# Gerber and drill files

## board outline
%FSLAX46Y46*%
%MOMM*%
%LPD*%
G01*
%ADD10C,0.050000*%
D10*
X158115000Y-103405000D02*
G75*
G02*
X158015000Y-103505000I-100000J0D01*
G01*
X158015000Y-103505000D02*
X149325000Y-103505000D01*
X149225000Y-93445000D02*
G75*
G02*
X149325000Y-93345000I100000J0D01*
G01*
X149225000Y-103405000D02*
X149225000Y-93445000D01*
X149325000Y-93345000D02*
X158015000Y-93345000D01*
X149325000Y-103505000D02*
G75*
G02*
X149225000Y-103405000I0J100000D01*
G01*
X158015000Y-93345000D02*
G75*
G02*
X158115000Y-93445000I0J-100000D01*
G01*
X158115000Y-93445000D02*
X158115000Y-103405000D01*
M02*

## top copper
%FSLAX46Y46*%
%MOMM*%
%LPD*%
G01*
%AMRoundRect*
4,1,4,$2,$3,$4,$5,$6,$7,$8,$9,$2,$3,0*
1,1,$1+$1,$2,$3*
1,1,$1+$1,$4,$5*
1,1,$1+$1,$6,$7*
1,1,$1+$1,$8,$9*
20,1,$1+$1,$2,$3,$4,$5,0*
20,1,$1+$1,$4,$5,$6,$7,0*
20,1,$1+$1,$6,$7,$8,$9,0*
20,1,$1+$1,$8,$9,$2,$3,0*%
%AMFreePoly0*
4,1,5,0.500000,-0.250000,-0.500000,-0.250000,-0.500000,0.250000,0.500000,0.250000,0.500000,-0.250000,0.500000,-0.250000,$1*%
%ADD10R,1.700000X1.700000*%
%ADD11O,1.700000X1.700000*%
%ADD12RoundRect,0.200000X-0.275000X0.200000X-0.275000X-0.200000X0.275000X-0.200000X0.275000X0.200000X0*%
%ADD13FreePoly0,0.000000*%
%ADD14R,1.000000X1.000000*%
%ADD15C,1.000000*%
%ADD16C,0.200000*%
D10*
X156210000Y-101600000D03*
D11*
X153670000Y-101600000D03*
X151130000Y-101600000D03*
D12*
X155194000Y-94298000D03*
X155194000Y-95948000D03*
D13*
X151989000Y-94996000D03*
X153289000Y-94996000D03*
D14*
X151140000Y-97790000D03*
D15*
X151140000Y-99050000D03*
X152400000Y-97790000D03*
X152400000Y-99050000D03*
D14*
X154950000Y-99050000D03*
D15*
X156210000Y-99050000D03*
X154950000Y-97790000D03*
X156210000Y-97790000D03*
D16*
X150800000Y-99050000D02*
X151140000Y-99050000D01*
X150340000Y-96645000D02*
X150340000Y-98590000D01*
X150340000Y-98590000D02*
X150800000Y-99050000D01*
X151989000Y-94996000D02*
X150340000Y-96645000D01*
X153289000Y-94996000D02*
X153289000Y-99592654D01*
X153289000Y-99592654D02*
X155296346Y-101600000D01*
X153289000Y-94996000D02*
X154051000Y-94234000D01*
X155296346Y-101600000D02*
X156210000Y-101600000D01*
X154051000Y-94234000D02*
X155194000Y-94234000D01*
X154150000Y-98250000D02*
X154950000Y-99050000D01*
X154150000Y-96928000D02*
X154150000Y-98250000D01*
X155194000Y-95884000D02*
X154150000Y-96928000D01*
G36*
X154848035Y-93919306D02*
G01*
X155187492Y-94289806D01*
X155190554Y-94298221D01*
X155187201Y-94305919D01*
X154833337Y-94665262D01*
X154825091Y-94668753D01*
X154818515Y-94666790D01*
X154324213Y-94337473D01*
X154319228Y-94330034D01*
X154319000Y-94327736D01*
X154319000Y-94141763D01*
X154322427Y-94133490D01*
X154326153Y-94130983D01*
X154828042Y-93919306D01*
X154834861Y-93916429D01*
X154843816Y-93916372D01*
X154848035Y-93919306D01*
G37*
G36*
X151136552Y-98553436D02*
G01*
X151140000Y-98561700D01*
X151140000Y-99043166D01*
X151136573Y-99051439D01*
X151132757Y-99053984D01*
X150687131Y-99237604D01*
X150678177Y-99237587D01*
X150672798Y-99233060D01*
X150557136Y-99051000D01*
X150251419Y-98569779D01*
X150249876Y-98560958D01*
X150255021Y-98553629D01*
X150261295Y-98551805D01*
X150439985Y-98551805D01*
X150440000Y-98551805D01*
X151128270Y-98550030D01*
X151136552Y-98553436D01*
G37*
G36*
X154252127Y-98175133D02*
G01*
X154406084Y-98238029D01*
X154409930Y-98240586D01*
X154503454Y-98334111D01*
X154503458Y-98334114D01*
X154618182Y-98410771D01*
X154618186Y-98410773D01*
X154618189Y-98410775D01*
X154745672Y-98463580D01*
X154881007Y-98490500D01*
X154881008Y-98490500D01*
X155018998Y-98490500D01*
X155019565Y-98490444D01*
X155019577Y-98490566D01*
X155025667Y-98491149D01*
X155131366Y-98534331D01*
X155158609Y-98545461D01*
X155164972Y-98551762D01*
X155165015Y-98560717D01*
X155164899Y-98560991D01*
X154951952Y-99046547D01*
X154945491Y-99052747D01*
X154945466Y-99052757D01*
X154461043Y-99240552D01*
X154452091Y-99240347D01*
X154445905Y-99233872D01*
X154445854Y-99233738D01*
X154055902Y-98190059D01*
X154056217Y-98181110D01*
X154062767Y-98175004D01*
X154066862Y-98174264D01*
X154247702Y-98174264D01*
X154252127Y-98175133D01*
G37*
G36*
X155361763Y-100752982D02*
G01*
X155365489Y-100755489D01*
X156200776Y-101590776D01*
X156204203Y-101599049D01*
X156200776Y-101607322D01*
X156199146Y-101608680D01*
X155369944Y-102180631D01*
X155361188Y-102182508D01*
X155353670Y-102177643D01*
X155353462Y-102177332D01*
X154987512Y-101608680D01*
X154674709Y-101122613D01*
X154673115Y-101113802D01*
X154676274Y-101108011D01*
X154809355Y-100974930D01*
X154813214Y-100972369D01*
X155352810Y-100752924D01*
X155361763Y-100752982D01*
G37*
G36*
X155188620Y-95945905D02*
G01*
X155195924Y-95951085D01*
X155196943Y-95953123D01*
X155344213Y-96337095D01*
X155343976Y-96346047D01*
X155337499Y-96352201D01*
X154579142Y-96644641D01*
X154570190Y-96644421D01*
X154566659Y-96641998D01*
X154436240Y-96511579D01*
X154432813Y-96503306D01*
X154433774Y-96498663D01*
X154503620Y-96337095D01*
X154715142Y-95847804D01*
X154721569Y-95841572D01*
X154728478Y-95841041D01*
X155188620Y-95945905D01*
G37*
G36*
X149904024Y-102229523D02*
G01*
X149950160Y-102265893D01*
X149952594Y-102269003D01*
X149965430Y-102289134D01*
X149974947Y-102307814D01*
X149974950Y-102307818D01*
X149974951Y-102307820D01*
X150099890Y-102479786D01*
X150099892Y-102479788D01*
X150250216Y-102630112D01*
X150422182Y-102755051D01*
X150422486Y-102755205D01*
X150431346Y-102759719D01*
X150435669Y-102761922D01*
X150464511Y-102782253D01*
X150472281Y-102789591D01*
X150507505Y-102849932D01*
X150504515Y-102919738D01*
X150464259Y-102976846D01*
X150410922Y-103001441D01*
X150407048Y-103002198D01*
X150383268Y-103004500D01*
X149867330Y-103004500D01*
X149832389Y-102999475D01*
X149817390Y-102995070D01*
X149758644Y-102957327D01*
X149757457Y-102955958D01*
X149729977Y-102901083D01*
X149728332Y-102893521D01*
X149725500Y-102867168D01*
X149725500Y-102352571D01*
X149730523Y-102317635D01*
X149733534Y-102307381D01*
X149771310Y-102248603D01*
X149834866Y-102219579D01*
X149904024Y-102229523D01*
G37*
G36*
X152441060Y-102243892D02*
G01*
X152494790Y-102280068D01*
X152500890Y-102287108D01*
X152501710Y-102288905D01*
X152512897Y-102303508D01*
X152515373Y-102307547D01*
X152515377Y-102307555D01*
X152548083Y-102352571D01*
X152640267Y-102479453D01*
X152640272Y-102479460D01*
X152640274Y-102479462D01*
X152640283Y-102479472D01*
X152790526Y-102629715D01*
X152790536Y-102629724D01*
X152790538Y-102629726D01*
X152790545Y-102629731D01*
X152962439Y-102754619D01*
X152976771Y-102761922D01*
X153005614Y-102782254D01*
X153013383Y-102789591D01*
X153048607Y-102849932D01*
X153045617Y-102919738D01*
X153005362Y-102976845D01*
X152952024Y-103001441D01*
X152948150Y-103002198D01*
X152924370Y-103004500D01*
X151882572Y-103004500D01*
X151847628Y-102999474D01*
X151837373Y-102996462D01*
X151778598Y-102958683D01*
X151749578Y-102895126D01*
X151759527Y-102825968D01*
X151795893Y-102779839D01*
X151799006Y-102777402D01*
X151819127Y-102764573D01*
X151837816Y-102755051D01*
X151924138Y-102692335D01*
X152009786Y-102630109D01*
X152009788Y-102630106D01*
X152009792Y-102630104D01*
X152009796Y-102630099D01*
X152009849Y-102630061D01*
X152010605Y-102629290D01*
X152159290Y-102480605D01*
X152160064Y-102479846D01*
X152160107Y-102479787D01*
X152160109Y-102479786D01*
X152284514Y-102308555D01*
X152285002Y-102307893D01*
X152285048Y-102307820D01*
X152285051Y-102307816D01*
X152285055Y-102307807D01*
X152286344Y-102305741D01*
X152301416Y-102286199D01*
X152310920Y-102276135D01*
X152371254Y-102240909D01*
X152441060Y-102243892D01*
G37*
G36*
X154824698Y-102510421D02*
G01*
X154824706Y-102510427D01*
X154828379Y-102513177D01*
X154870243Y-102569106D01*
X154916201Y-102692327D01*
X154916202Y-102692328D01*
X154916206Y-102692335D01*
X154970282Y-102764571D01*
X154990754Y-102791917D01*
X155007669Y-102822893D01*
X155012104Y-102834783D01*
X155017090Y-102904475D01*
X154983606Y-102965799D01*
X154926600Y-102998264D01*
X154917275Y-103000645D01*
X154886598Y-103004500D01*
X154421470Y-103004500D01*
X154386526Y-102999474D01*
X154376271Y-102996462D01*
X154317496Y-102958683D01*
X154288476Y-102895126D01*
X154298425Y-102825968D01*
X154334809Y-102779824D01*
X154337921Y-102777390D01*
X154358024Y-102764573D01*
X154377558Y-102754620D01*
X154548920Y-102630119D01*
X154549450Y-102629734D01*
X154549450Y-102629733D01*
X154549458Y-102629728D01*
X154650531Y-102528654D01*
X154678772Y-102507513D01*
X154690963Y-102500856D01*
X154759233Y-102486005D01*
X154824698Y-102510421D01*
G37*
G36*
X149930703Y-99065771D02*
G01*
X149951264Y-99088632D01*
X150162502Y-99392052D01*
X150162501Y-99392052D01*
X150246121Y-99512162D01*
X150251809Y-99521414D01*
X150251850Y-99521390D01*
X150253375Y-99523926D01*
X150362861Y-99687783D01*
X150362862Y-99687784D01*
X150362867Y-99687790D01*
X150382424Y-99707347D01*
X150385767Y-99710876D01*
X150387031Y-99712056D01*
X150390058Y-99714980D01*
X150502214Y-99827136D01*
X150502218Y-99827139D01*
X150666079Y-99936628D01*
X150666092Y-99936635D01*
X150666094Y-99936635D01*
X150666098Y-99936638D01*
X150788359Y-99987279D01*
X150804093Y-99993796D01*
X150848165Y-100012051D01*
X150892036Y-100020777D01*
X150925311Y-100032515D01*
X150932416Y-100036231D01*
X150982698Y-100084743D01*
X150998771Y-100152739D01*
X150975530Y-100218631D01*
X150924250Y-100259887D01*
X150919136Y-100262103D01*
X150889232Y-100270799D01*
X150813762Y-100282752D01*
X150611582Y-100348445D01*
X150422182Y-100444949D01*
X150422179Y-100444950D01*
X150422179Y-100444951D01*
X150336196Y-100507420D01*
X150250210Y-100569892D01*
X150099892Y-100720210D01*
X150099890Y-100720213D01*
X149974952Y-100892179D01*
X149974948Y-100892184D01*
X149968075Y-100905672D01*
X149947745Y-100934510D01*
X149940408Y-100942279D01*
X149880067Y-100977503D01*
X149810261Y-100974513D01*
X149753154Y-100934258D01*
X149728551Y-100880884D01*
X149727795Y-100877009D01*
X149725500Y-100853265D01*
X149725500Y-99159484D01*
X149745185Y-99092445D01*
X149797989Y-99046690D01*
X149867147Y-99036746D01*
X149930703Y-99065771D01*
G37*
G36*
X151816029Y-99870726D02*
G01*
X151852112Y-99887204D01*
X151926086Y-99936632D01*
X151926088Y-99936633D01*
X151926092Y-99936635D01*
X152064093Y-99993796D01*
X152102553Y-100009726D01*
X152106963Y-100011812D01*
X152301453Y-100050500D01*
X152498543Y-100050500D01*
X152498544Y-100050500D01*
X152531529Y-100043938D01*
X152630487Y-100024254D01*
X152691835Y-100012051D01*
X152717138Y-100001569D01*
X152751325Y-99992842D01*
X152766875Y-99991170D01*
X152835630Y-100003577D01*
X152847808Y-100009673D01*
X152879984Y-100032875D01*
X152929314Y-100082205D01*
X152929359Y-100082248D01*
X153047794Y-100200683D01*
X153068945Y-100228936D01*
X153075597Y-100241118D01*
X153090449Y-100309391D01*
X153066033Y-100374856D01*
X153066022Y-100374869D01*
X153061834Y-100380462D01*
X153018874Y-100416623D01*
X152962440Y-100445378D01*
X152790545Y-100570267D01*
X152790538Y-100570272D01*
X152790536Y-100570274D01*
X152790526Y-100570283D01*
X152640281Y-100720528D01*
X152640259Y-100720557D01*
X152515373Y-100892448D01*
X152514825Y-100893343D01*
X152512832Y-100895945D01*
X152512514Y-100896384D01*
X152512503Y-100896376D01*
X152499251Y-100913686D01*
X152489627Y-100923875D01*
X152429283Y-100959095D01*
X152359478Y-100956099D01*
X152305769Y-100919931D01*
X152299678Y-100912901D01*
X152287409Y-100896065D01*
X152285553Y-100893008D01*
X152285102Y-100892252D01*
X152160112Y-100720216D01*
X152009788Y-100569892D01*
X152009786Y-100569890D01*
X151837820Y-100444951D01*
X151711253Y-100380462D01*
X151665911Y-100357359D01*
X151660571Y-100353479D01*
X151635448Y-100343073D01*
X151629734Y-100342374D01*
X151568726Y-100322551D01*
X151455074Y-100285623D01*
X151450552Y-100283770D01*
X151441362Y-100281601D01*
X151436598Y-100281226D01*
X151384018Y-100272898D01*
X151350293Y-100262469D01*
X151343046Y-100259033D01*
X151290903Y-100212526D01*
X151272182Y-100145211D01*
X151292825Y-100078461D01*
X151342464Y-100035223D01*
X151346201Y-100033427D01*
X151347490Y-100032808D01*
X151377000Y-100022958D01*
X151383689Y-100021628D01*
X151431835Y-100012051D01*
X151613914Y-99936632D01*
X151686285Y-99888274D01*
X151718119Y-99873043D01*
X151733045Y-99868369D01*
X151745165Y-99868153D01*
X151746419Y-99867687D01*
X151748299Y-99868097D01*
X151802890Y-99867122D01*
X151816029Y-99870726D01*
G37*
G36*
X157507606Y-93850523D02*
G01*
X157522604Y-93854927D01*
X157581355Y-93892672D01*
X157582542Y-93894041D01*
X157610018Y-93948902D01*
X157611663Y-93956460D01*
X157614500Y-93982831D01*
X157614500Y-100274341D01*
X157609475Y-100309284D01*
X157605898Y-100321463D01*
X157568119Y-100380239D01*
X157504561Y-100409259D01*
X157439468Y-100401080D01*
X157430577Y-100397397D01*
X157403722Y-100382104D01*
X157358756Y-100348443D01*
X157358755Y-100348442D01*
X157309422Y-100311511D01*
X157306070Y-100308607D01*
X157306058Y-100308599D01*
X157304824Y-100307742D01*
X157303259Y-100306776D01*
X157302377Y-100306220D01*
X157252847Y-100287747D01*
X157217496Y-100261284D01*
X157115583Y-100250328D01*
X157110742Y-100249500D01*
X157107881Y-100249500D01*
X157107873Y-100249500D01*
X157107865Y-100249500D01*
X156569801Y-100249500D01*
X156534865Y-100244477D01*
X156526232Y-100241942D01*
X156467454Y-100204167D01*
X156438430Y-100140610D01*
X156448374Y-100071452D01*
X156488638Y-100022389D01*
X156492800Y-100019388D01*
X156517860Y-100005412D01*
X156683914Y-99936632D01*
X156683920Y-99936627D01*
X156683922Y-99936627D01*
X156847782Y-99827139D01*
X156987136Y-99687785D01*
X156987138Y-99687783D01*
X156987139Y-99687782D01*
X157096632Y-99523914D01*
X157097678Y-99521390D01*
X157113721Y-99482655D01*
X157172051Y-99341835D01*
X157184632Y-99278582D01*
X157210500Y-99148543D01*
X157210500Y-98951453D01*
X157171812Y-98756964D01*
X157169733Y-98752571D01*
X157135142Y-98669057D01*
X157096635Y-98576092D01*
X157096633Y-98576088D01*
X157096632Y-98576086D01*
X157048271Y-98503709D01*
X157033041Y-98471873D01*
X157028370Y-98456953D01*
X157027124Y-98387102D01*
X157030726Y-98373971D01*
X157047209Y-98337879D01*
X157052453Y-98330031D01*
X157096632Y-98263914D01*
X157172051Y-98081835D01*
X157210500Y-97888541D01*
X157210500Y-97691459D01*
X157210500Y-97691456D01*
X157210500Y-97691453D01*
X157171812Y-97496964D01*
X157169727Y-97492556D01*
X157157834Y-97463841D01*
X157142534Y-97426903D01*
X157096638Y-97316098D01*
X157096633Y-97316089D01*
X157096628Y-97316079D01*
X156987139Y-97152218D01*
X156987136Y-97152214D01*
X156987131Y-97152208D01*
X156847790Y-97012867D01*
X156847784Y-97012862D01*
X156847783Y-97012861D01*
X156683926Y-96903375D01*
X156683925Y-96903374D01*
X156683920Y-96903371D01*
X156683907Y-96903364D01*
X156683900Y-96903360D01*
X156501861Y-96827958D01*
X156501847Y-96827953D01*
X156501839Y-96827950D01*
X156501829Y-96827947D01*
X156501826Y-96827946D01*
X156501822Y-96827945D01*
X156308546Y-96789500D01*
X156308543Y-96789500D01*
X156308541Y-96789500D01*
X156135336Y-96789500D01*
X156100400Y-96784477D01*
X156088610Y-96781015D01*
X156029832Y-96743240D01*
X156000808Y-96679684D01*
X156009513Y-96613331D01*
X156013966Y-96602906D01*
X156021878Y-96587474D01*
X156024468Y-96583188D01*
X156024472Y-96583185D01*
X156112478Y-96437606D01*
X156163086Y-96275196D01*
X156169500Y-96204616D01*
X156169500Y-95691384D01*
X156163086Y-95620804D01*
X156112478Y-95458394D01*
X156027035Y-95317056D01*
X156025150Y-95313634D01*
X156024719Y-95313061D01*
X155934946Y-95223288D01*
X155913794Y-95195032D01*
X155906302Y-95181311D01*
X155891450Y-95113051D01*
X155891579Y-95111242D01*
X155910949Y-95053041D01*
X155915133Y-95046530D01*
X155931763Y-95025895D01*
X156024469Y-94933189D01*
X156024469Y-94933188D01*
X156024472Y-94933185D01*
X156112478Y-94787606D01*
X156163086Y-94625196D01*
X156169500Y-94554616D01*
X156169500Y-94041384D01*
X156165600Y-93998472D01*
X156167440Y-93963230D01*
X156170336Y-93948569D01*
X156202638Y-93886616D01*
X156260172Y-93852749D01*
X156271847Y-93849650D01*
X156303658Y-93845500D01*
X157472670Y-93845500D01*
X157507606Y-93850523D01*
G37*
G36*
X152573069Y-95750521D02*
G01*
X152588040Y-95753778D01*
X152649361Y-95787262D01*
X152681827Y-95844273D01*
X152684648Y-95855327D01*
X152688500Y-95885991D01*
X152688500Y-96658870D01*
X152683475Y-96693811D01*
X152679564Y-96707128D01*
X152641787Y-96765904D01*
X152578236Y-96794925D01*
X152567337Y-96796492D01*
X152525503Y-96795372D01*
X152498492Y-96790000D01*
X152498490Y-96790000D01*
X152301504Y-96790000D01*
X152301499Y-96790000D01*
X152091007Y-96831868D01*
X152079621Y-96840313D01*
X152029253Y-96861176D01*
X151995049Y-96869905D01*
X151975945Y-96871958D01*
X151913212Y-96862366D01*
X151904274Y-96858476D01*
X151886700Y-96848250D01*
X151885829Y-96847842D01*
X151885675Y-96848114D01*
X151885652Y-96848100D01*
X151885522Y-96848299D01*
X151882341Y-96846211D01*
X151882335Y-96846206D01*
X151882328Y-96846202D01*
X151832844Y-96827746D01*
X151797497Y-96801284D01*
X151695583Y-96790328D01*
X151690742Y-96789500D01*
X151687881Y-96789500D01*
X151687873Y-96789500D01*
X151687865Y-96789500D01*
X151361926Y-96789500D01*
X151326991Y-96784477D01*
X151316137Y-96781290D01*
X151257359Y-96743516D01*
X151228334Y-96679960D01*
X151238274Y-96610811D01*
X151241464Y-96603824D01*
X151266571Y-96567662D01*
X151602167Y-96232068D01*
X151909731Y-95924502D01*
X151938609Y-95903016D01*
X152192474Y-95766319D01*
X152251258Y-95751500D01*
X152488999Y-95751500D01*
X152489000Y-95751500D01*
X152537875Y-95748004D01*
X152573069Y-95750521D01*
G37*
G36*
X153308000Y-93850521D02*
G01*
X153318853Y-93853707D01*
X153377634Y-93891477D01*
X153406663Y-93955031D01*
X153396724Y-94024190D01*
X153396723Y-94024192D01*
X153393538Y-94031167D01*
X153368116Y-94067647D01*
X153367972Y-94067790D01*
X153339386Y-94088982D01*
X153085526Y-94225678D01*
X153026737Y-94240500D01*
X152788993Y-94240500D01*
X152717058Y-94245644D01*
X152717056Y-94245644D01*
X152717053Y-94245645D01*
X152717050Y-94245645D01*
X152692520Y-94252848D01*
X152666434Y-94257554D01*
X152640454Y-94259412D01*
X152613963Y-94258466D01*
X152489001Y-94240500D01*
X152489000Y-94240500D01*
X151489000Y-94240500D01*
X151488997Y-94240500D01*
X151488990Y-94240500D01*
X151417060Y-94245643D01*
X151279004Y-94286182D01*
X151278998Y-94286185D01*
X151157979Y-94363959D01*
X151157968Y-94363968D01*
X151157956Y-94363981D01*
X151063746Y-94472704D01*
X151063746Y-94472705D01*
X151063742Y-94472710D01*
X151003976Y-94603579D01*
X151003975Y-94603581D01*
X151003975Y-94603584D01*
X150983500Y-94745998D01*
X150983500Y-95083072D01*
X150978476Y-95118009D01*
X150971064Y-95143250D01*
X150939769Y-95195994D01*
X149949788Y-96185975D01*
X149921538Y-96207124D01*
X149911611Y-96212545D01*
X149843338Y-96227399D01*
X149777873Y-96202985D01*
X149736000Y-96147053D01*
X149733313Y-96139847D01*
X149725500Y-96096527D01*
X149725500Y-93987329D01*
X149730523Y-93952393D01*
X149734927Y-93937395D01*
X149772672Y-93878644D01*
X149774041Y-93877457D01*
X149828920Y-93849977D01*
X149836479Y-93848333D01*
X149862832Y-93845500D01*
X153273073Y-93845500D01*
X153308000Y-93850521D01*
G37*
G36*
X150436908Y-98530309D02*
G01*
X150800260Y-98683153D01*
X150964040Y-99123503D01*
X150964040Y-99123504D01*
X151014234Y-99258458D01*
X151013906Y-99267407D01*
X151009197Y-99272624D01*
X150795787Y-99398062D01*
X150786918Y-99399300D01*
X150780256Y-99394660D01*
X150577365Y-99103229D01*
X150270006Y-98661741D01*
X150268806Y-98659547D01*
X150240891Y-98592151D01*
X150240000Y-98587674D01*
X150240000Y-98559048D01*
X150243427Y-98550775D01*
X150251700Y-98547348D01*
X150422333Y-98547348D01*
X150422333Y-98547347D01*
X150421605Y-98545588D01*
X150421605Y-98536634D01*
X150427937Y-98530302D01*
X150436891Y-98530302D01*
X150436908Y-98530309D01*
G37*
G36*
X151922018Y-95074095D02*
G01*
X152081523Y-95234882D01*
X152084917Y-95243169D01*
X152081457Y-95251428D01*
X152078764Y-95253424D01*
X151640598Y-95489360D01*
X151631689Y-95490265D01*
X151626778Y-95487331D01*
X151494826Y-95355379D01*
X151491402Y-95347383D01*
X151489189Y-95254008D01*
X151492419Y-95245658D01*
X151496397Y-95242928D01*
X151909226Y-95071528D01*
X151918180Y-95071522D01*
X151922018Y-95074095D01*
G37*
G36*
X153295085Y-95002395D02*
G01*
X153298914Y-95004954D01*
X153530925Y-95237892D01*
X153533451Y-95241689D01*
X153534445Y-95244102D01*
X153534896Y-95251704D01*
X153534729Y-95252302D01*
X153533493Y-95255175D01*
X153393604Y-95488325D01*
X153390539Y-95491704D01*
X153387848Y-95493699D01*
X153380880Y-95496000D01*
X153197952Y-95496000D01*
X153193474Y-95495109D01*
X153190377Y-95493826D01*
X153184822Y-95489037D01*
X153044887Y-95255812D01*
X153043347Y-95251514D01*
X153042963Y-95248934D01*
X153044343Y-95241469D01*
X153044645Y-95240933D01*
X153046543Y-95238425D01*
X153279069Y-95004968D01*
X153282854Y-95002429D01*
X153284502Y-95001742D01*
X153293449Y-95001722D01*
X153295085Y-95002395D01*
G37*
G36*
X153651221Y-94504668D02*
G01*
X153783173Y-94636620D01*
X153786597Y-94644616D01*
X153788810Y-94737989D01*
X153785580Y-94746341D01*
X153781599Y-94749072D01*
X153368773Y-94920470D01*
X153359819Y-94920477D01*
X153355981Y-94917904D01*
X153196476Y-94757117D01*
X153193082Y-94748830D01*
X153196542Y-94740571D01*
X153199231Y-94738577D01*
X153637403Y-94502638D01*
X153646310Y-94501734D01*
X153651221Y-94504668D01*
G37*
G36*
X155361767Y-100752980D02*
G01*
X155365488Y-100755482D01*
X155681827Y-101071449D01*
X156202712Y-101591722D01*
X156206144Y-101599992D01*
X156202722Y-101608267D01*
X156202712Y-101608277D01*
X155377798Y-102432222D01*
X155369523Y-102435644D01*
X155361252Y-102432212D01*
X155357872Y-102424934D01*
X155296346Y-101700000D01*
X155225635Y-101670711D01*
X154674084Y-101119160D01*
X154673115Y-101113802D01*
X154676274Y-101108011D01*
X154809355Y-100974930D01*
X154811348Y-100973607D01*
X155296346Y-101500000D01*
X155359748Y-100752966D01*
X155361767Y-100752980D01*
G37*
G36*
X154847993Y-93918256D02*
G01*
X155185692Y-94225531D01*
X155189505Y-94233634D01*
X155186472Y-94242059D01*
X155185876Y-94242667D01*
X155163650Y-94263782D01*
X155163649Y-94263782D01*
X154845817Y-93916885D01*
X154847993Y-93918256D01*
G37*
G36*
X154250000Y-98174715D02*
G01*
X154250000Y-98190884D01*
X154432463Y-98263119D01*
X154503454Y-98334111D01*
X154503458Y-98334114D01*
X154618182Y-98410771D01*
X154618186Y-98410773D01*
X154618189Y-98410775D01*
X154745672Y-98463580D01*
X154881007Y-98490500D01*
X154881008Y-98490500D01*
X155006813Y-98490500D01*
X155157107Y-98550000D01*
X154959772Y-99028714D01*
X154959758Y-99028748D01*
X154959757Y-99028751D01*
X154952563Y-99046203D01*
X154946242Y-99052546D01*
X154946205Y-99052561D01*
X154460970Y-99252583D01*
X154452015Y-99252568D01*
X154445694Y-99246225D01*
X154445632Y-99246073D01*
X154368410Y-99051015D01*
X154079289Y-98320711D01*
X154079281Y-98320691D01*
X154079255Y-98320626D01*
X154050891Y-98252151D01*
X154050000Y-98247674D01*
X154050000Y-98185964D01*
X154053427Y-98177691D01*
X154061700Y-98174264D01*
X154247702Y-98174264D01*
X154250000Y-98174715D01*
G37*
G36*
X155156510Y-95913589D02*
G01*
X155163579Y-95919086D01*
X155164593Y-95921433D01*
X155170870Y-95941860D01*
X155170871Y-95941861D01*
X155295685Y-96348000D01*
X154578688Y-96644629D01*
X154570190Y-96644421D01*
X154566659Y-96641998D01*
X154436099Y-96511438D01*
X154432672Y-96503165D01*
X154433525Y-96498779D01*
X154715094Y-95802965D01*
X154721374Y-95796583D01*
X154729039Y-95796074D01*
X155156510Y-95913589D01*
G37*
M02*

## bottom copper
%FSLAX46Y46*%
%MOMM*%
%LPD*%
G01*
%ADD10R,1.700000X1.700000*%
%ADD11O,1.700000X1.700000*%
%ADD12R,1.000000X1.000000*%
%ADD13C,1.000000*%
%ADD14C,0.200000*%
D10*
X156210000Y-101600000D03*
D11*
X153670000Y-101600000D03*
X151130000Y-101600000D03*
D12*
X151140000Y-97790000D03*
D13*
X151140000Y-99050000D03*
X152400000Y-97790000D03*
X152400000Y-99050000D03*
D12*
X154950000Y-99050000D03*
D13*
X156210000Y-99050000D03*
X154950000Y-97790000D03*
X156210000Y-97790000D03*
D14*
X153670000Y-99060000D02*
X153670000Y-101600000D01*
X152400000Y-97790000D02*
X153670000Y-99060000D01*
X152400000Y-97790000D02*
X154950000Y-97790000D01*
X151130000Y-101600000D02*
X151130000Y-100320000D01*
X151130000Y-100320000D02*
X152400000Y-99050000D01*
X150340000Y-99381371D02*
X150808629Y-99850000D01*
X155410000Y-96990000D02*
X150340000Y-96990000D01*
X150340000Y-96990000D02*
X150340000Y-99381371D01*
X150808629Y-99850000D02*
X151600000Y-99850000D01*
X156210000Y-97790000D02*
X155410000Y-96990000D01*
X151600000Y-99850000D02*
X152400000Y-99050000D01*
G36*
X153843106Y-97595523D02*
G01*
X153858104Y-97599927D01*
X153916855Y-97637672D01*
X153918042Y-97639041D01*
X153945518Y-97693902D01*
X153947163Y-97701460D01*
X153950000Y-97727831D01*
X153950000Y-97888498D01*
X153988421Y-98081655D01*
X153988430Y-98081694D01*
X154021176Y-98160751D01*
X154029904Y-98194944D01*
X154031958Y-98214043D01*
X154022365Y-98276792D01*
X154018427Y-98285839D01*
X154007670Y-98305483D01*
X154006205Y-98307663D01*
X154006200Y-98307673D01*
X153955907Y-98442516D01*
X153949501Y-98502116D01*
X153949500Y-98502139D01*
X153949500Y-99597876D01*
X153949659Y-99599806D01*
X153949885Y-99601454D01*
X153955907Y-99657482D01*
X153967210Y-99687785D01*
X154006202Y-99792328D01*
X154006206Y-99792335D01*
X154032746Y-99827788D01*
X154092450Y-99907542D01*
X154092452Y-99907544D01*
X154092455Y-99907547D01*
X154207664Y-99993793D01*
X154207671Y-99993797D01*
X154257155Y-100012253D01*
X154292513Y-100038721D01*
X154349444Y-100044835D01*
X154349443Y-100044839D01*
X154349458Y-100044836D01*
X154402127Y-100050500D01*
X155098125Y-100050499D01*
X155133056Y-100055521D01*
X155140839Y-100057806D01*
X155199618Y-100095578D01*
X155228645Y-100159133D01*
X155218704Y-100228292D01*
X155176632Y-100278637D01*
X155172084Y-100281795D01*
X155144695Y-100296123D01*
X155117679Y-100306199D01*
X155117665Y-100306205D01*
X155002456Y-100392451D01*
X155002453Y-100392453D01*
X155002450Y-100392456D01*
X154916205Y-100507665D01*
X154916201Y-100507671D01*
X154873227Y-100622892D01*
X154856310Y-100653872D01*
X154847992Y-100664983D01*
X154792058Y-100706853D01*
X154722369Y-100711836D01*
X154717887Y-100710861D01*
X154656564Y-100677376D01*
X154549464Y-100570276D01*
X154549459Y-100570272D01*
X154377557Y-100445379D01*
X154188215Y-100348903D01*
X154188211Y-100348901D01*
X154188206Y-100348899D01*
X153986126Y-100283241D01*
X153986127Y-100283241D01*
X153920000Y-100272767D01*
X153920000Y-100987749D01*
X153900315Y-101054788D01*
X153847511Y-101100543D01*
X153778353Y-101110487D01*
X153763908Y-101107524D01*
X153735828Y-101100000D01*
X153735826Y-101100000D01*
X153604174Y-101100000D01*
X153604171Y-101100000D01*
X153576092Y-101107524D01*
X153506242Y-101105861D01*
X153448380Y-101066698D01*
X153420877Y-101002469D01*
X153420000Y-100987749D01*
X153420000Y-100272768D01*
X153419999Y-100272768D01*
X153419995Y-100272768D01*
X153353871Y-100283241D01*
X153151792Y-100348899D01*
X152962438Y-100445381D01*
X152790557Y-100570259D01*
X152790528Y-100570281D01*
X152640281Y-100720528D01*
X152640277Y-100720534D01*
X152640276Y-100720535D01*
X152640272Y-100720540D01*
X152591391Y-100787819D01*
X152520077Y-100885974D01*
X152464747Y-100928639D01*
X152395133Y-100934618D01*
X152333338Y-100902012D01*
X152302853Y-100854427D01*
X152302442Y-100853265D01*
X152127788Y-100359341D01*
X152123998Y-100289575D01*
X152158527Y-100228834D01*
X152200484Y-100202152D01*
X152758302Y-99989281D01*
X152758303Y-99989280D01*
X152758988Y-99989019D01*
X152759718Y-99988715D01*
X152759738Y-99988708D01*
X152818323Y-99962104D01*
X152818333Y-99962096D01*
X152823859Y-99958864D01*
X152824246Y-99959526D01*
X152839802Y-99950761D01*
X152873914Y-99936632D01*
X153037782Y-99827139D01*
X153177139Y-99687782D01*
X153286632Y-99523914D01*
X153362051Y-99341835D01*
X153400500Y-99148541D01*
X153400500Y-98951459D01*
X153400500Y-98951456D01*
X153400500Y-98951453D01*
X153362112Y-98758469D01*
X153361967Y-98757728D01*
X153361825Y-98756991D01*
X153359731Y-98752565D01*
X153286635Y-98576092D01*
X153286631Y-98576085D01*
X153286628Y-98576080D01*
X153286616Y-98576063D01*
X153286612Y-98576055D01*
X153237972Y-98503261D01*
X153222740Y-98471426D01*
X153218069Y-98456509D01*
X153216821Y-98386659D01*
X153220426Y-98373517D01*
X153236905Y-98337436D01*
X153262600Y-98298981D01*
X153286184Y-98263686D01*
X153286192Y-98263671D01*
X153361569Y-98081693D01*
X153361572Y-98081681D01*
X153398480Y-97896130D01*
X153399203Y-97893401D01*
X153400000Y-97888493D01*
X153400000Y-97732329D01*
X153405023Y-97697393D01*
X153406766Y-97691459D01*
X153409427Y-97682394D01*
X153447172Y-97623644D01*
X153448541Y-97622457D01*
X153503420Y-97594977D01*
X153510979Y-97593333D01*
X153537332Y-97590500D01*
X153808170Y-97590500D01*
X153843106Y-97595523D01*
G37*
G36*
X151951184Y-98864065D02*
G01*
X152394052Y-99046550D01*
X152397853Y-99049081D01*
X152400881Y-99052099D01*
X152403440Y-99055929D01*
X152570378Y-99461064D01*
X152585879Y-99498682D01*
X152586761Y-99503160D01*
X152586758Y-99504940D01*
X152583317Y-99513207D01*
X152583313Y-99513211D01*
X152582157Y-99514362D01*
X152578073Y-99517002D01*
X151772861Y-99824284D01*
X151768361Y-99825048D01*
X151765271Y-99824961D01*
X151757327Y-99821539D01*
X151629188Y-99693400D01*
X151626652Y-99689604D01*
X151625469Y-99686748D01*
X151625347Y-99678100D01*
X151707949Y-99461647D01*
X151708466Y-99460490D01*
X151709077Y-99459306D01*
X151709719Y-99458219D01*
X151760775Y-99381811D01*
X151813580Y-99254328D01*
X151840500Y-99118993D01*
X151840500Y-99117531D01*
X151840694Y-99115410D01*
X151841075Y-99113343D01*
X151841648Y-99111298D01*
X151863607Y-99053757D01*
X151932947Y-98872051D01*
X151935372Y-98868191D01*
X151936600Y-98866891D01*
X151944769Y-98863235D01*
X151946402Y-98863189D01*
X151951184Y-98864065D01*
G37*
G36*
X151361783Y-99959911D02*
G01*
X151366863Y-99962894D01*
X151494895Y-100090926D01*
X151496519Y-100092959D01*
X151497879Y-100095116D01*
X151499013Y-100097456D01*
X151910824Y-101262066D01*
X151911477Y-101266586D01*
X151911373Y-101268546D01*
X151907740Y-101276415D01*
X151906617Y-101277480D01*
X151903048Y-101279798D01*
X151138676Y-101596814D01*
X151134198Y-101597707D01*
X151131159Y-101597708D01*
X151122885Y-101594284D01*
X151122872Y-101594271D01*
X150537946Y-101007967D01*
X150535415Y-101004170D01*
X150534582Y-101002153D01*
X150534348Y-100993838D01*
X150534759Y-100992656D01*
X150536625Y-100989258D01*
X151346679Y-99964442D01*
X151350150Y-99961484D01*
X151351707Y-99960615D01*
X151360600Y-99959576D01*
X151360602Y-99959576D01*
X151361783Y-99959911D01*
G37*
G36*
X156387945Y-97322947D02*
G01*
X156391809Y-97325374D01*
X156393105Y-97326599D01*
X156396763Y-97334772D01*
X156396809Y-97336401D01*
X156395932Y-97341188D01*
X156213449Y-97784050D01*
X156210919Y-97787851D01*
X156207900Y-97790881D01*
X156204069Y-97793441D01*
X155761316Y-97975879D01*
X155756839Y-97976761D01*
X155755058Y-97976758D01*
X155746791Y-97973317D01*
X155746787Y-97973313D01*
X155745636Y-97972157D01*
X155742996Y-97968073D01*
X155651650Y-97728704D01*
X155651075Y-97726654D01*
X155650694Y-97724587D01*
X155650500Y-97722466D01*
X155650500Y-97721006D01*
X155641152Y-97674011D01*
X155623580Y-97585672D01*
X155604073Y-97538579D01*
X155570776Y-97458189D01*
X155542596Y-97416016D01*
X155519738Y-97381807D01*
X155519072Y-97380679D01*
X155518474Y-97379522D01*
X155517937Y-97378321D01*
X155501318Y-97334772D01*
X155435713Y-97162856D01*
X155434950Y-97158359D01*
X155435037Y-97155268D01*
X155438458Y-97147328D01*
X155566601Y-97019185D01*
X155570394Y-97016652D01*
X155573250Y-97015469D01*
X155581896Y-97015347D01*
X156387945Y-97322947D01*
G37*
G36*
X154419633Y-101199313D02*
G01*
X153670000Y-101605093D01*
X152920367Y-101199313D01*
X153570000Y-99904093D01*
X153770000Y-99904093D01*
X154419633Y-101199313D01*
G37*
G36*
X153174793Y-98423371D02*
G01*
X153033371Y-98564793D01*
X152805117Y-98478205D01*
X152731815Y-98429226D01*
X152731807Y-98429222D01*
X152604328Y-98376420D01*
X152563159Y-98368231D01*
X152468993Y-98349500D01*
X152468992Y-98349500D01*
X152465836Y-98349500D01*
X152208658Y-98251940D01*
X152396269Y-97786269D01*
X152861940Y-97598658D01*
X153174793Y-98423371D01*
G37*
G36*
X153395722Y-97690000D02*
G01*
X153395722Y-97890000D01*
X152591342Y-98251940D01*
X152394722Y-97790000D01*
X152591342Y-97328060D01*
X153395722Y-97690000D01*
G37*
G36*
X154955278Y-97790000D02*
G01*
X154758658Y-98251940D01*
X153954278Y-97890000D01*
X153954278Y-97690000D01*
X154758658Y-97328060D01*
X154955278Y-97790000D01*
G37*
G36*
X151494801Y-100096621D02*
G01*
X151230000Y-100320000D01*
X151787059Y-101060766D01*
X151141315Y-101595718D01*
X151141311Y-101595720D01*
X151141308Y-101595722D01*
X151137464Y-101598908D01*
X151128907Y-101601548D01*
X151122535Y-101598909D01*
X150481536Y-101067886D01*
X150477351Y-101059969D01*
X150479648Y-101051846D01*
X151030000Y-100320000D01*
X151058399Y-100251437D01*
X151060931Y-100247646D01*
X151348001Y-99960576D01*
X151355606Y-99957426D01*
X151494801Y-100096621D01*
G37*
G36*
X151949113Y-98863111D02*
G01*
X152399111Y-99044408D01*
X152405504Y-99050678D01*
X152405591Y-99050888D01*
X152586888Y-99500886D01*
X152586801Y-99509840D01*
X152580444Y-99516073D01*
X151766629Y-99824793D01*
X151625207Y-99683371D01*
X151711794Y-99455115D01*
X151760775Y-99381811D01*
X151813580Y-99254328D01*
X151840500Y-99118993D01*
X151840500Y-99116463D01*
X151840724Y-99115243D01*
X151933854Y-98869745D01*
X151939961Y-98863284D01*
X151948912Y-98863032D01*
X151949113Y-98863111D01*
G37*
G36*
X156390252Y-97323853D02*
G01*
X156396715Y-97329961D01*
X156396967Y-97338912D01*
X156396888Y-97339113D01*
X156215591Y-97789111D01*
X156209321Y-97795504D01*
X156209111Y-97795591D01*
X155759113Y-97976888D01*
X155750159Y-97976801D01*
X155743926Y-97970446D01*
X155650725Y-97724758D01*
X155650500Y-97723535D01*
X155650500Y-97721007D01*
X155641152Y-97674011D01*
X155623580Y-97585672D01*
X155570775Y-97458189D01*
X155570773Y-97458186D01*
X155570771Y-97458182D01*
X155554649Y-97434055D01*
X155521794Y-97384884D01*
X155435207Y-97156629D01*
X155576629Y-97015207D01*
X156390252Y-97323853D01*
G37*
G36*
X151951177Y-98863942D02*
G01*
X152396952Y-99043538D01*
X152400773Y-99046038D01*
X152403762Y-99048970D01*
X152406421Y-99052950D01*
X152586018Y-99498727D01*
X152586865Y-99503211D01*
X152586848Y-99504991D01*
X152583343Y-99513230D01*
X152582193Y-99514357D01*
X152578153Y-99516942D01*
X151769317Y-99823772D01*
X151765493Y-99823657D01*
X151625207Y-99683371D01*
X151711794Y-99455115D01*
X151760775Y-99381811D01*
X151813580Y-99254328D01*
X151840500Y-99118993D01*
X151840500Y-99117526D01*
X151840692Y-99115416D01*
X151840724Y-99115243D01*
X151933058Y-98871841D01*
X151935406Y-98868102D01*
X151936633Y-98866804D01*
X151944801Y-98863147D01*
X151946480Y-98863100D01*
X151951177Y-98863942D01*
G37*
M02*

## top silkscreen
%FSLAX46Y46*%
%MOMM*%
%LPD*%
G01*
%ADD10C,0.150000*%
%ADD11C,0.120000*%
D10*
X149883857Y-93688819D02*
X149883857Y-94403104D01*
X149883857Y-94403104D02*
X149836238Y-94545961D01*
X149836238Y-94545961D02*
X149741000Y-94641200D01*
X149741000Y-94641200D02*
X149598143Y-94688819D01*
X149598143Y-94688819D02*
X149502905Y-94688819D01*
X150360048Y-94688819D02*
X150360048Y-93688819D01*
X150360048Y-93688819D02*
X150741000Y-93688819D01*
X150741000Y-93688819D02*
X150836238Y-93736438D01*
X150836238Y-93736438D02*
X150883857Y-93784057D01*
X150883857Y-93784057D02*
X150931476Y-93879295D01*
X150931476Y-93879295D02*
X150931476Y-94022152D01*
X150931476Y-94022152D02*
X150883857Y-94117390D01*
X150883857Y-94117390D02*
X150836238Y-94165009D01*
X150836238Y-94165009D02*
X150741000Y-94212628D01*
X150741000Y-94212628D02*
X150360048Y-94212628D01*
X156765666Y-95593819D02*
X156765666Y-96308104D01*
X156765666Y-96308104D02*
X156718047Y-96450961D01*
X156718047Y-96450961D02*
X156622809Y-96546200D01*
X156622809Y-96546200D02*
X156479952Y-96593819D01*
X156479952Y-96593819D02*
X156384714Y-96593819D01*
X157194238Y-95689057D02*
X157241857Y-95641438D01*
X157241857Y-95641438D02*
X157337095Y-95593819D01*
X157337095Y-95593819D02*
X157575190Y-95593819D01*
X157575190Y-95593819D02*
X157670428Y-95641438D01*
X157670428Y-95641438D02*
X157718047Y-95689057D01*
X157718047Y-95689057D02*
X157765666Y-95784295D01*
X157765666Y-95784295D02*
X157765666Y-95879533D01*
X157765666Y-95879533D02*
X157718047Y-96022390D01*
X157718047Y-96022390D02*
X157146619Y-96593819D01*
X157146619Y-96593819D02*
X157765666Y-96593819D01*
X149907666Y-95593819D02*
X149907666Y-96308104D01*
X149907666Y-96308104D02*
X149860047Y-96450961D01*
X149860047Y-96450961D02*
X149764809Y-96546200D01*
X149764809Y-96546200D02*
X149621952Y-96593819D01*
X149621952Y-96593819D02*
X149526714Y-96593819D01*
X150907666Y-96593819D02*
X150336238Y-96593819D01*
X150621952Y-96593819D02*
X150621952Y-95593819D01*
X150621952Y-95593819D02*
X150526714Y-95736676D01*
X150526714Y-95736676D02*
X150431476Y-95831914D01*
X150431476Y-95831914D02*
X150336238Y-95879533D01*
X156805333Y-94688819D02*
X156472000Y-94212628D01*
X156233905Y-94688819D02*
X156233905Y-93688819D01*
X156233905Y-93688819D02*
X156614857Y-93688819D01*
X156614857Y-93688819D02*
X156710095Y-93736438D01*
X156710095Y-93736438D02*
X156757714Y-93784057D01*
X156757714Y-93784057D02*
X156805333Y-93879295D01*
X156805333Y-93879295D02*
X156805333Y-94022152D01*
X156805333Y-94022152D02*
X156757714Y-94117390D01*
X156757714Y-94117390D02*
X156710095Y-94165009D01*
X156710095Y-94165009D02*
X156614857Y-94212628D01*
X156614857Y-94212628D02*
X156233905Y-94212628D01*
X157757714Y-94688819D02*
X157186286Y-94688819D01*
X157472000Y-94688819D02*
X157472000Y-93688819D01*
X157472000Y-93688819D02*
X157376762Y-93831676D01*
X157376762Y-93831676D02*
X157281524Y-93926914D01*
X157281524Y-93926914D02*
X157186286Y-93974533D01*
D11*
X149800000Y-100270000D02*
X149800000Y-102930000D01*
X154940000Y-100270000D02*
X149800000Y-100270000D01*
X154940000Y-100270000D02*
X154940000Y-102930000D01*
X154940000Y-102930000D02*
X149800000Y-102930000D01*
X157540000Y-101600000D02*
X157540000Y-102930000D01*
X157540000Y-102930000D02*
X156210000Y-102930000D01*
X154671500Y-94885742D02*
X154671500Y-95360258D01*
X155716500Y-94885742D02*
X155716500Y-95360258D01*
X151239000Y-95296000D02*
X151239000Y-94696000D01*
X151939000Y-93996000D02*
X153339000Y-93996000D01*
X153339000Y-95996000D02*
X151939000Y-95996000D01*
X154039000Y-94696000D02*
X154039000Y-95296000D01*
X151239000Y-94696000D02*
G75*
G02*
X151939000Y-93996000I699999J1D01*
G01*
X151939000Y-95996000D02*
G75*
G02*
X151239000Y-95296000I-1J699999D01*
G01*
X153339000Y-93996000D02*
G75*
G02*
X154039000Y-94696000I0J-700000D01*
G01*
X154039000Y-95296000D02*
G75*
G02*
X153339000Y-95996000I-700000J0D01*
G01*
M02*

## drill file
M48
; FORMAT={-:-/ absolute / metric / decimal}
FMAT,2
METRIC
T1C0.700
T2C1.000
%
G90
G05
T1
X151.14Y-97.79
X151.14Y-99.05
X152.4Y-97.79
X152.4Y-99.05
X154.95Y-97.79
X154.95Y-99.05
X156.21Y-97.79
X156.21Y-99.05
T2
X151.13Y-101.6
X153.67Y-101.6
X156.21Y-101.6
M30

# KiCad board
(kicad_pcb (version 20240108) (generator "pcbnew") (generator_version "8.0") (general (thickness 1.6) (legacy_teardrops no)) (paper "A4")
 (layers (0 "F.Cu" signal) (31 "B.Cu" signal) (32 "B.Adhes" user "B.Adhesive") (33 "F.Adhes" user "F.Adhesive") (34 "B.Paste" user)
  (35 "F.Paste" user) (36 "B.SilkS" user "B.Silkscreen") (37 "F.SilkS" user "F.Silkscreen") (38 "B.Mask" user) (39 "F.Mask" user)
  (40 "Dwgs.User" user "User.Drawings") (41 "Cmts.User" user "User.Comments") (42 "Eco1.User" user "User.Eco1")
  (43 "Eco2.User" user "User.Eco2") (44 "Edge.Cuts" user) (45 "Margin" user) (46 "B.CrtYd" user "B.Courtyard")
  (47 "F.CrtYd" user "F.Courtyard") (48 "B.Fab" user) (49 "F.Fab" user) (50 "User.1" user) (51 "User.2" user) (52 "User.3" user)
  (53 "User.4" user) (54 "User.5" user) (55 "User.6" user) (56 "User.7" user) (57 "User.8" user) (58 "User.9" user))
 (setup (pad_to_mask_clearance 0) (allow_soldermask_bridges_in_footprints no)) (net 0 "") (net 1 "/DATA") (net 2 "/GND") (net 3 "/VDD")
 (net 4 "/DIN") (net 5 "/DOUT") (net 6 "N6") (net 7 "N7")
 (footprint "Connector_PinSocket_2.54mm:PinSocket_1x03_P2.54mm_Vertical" (layer "F.Cu") (at 156.21 101.6 -90)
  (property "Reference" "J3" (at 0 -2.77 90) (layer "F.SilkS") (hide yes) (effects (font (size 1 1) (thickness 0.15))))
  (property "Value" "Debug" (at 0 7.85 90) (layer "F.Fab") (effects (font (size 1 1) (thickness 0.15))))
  (fp_line (start -1.33 6.41) (end 1.33 6.41) (stroke (width 0.12) (type solid)) (layer "F.SilkS"))
  (fp_line (start -1.33 1.27) (end -1.33 6.41) (stroke (width 0.12) (type solid)) (layer "F.SilkS"))
  (fp_line (start -1.33 1.27) (end 1.33 1.27) (stroke (width 0.12) (type solid)) (layer "F.SilkS"))
  (fp_line (start 1.33 1.27) (end 1.33 6.41) (stroke (width 0.12) (type solid)) (layer "F.SilkS"))
  (fp_line (start 0 -1.33) (end 1.33 -1.33) (stroke (width 0.12) (type solid)) (layer "F.SilkS"))
  (fp_line (start 1.33 -1.33) (end 1.33 0) (stroke (width 0.12) (type solid)) (layer "F.SilkS"))
  (pad "1" thru_hole rect (at 0 0 270) (size 1.7 1.7) (drill 1) (layers "*.Cu" "*.Mask") (remove_unused_layers no) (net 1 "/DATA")
   (teardrops (best_length_ratio 0.5) (max_length 1) (best_width_ratio 1) (max_width 2) (curve_points 0) (filter_ratio 0.9) (enabled yes)
    (allow_two_segments yes) (prefer_zone_connections yes)))
  (pad "2" thru_hole oval (at 0 2.54 270) (size 1.7 1.7) (drill 1) (layers "*.Cu" "*.Mask") (remove_unused_layers no) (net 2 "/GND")
   (teardrops (best_length_ratio 0.5) (max_length 1) (best_width_ratio 1) (max_width 2) (curve_points 0) (filter_ratio 0.9) (enabled yes)
    (allow_two_segments yes) (prefer_zone_connections yes)))
  (pad "3" thru_hole oval (at 0 5.08 270) (size 1.7 1.7) (drill 1) (layers "*.Cu" "*.Mask") (remove_unused_layers no) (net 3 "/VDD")
   (teardrops (best_length_ratio 0.5) (max_length 1) (best_width_ratio 1) (max_width 2) (curve_points 0) (filter_ratio 0.9) (enabled yes)
    (allow_two_segments yes) (prefer_zone_connections yes))))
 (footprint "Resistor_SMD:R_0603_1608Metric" (layer "F.Cu") (at 155.194 95.123 -90)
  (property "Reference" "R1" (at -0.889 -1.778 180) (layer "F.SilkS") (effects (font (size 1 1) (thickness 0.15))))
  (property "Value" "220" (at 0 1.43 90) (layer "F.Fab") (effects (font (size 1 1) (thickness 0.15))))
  (fp_line (start -0.237258 0.5225) (end 0.237258 0.5225) (stroke (width 0.12) (type solid)) (layer "F.SilkS"))
  (fp_line (start -0.237258 -0.5225) (end 0.237258 -0.5225) (stroke (width 0.12) (type solid)) (layer "F.SilkS"))
  (pad "1" smd roundrect (at -0.825 0 270) (size 0.8 0.95) (layers "F.Cu" "F.Paste" "F.Mask") (roundrect_rratio 0.25) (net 1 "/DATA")
   (teardrops (best_length_ratio 0.5) (max_length 1) (best_width_ratio 1) (max_width 2) (curve_points 0) (filter_ratio 0.9) (enabled yes)
    (allow_two_segments yes) (prefer_zone_connections yes)))
  (pad "2" smd roundrect (at 0.825 0 270) (size 0.8 0.95) (layers "F.Cu" "F.Paste" "F.Mask") (roundrect_rratio 0.25) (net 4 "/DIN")
   (teardrops (best_length_ratio 0.5) (max_length 1) (best_width_ratio 1) (max_width 2) (curve_points 0) (filter_ratio 0.9) (enabled yes)
    (allow_two_segments yes) (prefer_zone_connections yes))))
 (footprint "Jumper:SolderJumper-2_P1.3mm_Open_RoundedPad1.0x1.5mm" (layer "F.Cu") (at 152.639 94.996)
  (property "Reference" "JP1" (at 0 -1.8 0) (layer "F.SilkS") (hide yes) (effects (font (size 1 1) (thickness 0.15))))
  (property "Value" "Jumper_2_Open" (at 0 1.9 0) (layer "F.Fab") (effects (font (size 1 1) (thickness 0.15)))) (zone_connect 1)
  (fp_line (start -1.4 0.3) (end -1.4 -0.3) (stroke (width 0.12) (type solid)) (layer "F.SilkS"))
  (fp_line (start -0.7 -1) (end 0.7 -1) (stroke (width 0.12) (type solid)) (layer "F.SilkS"))
  (fp_line (start 0.7 1) (end -0.7 1) (stroke (width 0.12) (type solid)) (layer "F.SilkS"))
  (fp_line (start 1.4 -0.3) (end 1.4 0.3) (stroke (width 0.12) (type solid)) (layer "F.SilkS"))
  (fp_arc (start -1.4 -0.3) (mid -1.194975 -0.794975) (end -0.7 -1) (stroke (width 0.12) (type solid)) (layer "F.SilkS"))
  (fp_arc (start -0.7 1) (mid -1.194975 0.794975) (end -1.4 0.3) (stroke (width 0.12) (type solid)) (layer "F.SilkS"))
  (fp_arc (start 0.7 -1) (mid 1.194975 -0.794975) (end 1.4 -0.3) (stroke (width 0.12) (type solid)) (layer "F.SilkS"))
  (fp_arc (start 1.4 0.3) (mid 1.194975 0.794975) (end 0.7 1) (stroke (width 0.12) (type solid)) (layer "F.SilkS"))
  (pad "1" smd custom (at -0.65 0) (size 1 0.5) (layers "F.Cu" "F.Mask") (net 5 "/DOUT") (zone_connect 2) (thermal_bridge_angle 45)
   (options (clearance outline) (anchor rect)) (primitives)
   (teardrops (best_length_ratio 0.5) (max_length 1) (best_width_ratio 1) (max_width 2) (curve_points 0) (filter_ratio 0.9) (enabled yes)
    (allow_two_segments yes) (prefer_zone_connections yes)))
  (pad "2" smd custom (at 0.65 0) (size 1 0.5) (layers "F.Cu" "F.Mask") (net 1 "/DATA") (zone_connect 2) (thermal_bridge_angle 45)
   (options (clearance outline) (anchor rect)) (primitives)
   (teardrops (best_length_ratio 0.5) (max_length 1) (best_width_ratio 1) (max_width 2) (curve_points 0) (filter_ratio 0.9) (enabled yes)
    (allow_two_segments yes) (prefer_zone_connections yes))))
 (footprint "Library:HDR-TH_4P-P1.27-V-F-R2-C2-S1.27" (layer "B.Cu") (at 151.77 98.42)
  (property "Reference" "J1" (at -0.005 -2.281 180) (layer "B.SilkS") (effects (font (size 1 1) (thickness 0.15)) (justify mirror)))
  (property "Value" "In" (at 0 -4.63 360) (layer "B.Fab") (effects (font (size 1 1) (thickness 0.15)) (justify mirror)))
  (pad "1" thru_hole rect (at -0.63 -0.63) (size 1 1) (drill 0.700024) (layers "*.Cu" "*.Mask") (remove_unused_layers no) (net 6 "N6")
   (teardrops (best_length_ratio 0.5) (max_length 1) (best_width_ratio 1) (max_width 2) (curve_points 0) (filter_ratio 0.9) (enabled yes)
    (allow_two_segments yes) (prefer_zone_connections yes)))
  (pad "2" thru_hole circle (at -0.63 0.63) (size 1 1) (drill 0.700024) (layers "*.Cu" "*.Mask") (remove_unused_layers no) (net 5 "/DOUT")
   (teardrops (best_length_ratio 0.5) (max_length 1) (best_width_ratio 1) (max_width 2) (curve_points 0) (filter_ratio 0.9) (enabled yes)
    (allow_two_segments yes) (prefer_zone_connections yes)))
  (pad "3" thru_hole circle (at 0.63 -0.63) (size 1 1) (drill 0.700024) (layers "*.Cu" "*.Mask") (remove_unused_layers no) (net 2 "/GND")
   (teardrops (best_length_ratio 0.5) (max_length 1) (best_width_ratio 1) (max_width 2) (curve_points 0) (filter_ratio 0.9) (enabled yes)
    (allow_two_segments yes) (prefer_zone_connections yes)))
  (pad "4" thru_hole circle (at 0.63 0.63) (size 1 1) (drill 0.700024) (layers "*.Cu" "*.Mask") (remove_unused_layers no) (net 3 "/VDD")
   (teardrops (best_length_ratio 0.5) (max_length 1) (best_width_ratio 1) (max_width 2) (curve_points 0) (filter_ratio 0.9) (enabled yes)
    (allow_two_segments yes) (prefer_zone_connections yes))))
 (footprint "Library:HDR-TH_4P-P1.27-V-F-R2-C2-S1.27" (layer "B.Cu") (at 155.58 98.42 90)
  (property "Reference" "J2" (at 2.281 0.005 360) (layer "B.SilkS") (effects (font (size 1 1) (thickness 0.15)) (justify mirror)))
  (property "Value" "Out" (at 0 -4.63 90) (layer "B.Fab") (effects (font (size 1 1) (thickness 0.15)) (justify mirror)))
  (pad "1" thru_hole rect (at -0.63 -0.63 90) (size 1 1) (drill 0.700024) (layers "*.Cu" "*.Mask") (remove_unused_layers no) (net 4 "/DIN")
   (teardrops (best_length_ratio 0.5) (max_length 1) (best_width_ratio 1) (max_width 2) (curve_points 0) (filter_ratio 0.9) (enabled yes)
    (allow_two_segments yes) (prefer_zone_connections yes)))
  (pad "2" thru_hole circle (at -0.63 0.63 90) (size 1 1) (drill 0.700024) (layers "*.Cu" "*.Mask") (remove_unused_layers no) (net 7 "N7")
   (teardrops (best_length_ratio 0.5) (max_length 1) (best_width_ratio 1) (max_width 2) (curve_points 0) (filter_ratio 0.9) (enabled yes)
    (allow_two_segments yes) (prefer_zone_connections yes)))
  (pad "3" thru_hole circle (at 0.63 -0.63 90) (size 1 1) (drill 0.700024) (layers "*.Cu" "*.Mask") (remove_unused_layers no) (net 2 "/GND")
   (teardrops (best_length_ratio 0.5) (max_length 1) (best_width_ratio 1) (max_width 2) (curve_points 0) (filter_ratio 0.9) (enabled yes)
    (allow_two_segments yes) (prefer_zone_connections yes)))
  (pad "4" thru_hole circle (at 0.63 0.63 90) (size 1 1) (drill 0.700024) (layers "*.Cu" "*.Mask") (remove_unused_layers no) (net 3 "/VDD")
   (teardrops (best_length_ratio 0.5) (max_length 1) (best_width_ratio 1) (max_width 2) (curve_points 0) (filter_ratio 0.9) (enabled yes)
    (allow_two_segments yes) (prefer_zone_connections yes))))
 (gr_arc (start 158.115 103.405) (mid 158.085711 103.475711) (end 158.015 103.505) (stroke (width 0.05) (type default)) (layer "Edge.Cuts"))
 (gr_line (start 158.015 103.505) (end 149.325 103.505) (stroke (width 0.05) (type default)) (layer "Edge.Cuts"))
 (gr_arc (start 149.225 93.445) (mid 149.254289 93.374289) (end 149.325 93.345) (stroke (width 0.05) (type default)) (layer "Edge.Cuts"))
 (gr_line (start 149.225 103.405) (end 149.225 93.445) (stroke (width 0.05) (type default)) (layer "Edge.Cuts"))
 (gr_line (start 149.325 93.345) (end 158.015 93.345) (stroke (width 0.05) (type default)) (layer "Edge.Cuts"))
 (gr_arc (start 149.325 103.505) (mid 149.254289 103.475711) (end 149.225 103.405) (stroke (width 0.05) (type default)) (layer "Edge.Cuts"))
 (gr_arc (start 158.015 93.345) (mid 158.085711 93.374289) (end 158.115 93.445) (stroke (width 0.05) (type default)) (layer "Edge.Cuts"))
 (gr_line (start 158.115 93.445) (end 158.115 103.405) (stroke (width 0.05) (type default)) (layer "Edge.Cuts"))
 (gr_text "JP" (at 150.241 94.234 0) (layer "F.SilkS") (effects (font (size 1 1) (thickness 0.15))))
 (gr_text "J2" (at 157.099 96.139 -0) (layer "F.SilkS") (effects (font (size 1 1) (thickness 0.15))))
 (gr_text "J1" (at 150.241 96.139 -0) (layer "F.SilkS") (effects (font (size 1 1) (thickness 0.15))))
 (segment (start 150.8 99.05) (end 151.14 99.05) (width 0.2) (layer "F.Cu") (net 5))
 (segment (start 150.34 96.645) (end 150.34 98.59) (width 0.2) (layer "F.Cu") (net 5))
 (segment (start 150.34 98.59) (end 150.8 99.05) (width 0.2) (layer "F.Cu") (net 5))
 (segment (start 151.989 94.996) (end 150.34 96.645) (width 0.2) (layer "F.Cu") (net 5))
 (segment (start 153.289 94.996) (end 153.289 99.592654) (width 0.2) (layer "F.Cu") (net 1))
 (segment (start 153.289 99.592654) (end 155.296346 101.6) (width 0.2) (layer "F.Cu") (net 1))
 (segment (start 153.289 94.996) (end 154.051 94.234) (width 0.2) (layer "F.Cu") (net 1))
 (segment (start 155.296346 101.6) (end 156.21 101.6) (width 0.2) (layer "F.Cu") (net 1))
 (segment (start 154.051 94.234) (end 155.194 94.234) (width 0.2) (layer "F.Cu") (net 1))
 (segment (start 154.15 98.25) (end 154.95 99.05) (width 0.2) (layer "F.Cu") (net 4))
 (segment (start 154.15 96.928) (end 154.15 98.25) (width 0.2) (layer "F.Cu") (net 4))
 (segment (start 155.194 95.884) (end 154.15 96.928) (width 0.2) (layer "F.Cu") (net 4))
 (segment (start 153.67 99.06) (end 153.67 101.6) (width 0.2) (layer "B.Cu") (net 2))
 (segment (start 152.4 97.79) (end 153.67 99.06) (width 0.2) (layer "B.Cu") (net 2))
 (segment (start 152.4 97.79) (end 154.95 97.79) (width 0.2) (layer "B.Cu") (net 2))
 (segment (start 151.13 101.6) (end 151.13 100.32) (width 0.2) (layer "B.Cu") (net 3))
 (segment (start 151.13 100.32) (end 152.4 99.05) (width 0.2) (layer "B.Cu") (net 3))
 (segment (start 150.34 99.381371) (end 150.808629 99.85) (width 0.2) (layer "B.Cu") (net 3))
 (segment (start 155.41 96.99) (end 150.34 96.99) (width 0.2) (layer "B.Cu") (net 3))
 (segment (start 150.34 96.99) (end 150.34 99.381371) (width 0.2) (layer "B.Cu") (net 3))
 (segment (start 150.808629 99.85) (end 151.6 99.85) (width 0.2) (layer "B.Cu") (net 3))
 (segment (start 156.21 97.79) (end 155.41 96.99) (width 0.2) (layer "B.Cu") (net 3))
 (segment (start 151.6 99.85) (end 152.4 99.05) (width 0.2) (layer "B.Cu") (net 3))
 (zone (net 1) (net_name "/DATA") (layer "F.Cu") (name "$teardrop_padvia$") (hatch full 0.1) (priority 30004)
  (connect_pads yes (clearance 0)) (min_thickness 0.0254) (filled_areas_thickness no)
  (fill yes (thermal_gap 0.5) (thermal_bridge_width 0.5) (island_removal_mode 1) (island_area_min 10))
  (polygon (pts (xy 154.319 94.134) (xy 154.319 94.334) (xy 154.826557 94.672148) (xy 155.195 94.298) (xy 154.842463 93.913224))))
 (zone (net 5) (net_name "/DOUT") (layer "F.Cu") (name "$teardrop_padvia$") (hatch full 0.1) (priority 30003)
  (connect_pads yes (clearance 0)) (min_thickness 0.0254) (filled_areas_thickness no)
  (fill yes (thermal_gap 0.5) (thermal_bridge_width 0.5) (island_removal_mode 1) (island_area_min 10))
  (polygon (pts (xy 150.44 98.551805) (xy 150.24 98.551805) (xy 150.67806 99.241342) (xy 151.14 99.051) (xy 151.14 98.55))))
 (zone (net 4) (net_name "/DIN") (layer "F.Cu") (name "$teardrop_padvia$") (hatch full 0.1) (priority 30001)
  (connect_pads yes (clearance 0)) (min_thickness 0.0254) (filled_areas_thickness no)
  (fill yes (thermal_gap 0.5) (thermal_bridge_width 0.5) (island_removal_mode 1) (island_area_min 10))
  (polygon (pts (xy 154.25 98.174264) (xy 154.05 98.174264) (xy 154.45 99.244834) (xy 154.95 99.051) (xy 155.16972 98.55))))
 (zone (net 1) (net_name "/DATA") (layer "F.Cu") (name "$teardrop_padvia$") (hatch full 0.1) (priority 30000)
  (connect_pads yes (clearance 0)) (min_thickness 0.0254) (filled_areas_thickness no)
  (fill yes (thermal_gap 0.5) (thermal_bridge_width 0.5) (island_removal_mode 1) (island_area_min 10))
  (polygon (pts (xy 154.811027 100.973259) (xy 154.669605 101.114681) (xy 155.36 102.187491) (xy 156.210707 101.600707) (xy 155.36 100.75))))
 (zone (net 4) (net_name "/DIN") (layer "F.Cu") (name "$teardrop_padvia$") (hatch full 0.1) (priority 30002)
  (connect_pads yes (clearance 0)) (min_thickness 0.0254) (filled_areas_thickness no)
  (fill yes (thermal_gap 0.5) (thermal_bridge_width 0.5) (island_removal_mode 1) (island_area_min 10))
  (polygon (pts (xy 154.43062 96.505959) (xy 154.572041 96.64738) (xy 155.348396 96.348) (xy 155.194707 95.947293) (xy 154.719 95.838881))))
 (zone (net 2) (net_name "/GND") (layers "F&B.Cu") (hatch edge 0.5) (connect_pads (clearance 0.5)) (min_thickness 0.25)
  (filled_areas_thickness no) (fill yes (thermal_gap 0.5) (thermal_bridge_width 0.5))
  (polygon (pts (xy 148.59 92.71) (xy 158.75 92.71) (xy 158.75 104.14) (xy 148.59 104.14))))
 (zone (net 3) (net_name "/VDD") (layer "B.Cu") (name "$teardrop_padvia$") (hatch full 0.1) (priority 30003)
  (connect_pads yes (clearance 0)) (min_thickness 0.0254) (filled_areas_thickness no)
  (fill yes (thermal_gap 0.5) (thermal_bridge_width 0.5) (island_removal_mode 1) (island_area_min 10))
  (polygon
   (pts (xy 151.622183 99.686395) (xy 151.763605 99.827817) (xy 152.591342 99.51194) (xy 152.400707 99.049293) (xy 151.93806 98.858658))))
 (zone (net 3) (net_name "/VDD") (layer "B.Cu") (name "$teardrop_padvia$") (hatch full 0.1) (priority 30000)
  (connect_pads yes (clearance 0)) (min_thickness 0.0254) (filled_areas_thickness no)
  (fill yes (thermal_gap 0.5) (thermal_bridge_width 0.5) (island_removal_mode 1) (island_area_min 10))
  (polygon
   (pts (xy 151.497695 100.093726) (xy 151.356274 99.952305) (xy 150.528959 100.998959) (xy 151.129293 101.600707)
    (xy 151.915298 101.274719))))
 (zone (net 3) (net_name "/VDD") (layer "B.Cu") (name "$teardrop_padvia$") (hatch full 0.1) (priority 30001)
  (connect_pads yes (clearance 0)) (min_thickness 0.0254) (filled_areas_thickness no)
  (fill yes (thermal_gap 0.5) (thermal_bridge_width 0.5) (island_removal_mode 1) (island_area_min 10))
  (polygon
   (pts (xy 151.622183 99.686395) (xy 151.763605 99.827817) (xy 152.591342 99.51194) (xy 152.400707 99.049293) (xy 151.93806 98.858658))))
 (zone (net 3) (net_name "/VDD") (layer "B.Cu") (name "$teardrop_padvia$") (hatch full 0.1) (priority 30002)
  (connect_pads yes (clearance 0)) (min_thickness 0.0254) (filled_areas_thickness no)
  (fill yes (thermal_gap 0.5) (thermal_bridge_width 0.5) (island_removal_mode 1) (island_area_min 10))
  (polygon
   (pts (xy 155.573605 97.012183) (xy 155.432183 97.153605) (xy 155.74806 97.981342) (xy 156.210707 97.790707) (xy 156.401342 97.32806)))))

